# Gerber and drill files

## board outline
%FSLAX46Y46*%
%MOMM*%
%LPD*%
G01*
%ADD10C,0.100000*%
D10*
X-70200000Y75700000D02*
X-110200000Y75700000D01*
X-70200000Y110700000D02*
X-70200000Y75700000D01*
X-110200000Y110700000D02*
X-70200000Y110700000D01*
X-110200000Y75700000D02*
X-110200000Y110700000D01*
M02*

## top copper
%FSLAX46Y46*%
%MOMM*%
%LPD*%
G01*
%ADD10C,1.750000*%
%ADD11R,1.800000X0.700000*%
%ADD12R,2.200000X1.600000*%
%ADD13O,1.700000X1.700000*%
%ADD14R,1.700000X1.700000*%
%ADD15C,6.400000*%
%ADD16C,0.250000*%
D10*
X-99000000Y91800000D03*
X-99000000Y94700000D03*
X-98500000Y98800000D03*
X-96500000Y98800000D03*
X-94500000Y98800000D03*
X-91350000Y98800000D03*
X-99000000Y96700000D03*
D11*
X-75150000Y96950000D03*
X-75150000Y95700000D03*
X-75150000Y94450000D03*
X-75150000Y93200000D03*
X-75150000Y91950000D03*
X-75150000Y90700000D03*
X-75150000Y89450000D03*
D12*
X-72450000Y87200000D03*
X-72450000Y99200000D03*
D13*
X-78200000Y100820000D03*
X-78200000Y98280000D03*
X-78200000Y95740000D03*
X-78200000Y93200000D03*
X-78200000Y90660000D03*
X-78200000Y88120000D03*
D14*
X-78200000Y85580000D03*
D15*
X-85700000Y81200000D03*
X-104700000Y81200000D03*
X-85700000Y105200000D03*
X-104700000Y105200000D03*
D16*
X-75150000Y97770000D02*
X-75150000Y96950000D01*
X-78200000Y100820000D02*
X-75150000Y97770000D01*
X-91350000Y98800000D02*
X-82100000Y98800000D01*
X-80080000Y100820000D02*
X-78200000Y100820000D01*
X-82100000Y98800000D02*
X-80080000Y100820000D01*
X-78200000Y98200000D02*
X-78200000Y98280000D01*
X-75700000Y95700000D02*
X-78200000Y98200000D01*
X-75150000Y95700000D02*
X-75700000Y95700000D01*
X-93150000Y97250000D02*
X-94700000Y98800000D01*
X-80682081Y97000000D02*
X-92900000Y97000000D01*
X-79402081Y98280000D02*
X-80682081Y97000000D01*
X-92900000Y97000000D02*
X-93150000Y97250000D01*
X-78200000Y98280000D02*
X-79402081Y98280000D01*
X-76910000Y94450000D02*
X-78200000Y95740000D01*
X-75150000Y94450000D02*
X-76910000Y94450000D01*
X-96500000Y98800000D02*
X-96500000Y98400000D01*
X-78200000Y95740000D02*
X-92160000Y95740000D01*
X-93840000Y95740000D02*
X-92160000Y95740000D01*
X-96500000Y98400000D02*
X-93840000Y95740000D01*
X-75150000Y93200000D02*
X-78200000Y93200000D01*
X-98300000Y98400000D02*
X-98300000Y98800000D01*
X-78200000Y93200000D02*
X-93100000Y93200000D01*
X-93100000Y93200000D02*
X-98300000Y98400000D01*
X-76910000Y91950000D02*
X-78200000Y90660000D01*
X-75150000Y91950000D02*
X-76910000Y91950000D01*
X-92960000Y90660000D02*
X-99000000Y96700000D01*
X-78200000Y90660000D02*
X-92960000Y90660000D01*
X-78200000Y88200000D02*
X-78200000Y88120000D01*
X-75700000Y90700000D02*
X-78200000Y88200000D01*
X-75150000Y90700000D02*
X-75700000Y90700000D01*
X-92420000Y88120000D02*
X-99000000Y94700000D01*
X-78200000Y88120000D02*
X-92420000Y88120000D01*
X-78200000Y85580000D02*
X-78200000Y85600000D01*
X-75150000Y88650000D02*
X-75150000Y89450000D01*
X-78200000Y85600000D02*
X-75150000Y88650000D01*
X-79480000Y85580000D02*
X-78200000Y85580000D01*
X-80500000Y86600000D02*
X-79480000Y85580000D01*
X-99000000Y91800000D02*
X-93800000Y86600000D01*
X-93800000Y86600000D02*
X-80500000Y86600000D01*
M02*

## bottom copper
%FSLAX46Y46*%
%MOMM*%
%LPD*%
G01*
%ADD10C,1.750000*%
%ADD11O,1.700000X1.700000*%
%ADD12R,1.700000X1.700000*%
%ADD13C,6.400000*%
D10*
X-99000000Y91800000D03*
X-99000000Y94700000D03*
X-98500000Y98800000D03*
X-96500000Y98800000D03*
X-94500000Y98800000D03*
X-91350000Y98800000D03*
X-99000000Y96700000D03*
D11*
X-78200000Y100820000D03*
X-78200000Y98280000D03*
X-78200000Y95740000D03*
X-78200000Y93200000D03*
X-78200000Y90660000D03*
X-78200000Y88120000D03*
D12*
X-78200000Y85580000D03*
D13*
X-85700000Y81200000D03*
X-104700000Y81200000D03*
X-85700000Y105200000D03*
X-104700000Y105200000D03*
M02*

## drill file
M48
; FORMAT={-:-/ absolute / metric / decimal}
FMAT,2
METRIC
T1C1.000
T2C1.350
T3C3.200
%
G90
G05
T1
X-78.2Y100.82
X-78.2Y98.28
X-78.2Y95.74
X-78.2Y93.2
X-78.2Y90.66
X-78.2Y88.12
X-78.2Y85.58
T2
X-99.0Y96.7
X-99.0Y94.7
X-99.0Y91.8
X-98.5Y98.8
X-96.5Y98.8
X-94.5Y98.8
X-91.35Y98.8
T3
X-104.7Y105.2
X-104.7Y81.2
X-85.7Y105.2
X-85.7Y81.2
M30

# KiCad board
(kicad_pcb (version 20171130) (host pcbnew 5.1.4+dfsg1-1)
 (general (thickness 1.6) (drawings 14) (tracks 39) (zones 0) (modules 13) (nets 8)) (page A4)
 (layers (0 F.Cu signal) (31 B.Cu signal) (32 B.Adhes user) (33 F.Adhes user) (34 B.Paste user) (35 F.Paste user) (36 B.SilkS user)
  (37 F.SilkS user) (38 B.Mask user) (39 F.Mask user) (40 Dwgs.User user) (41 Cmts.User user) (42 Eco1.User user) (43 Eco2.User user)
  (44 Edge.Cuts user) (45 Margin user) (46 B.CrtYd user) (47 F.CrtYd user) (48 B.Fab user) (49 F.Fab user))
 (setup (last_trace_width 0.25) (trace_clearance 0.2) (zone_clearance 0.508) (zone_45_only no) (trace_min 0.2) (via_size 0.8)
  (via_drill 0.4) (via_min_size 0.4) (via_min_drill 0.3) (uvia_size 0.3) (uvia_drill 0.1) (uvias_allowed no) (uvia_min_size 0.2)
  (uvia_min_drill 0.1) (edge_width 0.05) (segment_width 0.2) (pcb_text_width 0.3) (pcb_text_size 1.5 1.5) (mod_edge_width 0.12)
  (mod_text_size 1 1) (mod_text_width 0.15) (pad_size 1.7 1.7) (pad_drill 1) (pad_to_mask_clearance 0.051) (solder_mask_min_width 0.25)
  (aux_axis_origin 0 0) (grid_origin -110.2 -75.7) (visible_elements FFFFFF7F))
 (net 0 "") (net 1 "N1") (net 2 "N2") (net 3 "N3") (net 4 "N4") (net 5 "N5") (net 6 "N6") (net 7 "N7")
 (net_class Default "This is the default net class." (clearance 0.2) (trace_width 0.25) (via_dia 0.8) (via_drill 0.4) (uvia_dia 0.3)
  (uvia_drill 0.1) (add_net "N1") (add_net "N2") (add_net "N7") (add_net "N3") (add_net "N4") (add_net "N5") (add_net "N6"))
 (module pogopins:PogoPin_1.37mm (layer F.Cu) (at -99 -91.8)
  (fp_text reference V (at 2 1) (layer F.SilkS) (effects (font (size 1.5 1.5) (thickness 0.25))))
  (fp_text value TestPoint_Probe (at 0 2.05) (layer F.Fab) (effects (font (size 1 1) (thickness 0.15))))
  (pad 1 thru_hole circle (at 0 0) (size 1.75 1.75) (drill 1.35) (layers *.Cu *.Mask) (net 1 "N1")))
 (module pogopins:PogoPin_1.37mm (layer F.Cu) (at -99 -94.7)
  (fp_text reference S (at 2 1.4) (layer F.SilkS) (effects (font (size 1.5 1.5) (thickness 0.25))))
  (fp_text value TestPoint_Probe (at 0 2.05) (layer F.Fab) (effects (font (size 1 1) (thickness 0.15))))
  (pad 1 thru_hole circle (at 0 0) (size 1.75 1.75) (drill 1.35) (layers *.Cu *.Mask) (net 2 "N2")))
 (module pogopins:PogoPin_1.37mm (layer F.Cu) (at -98.5 -98.8)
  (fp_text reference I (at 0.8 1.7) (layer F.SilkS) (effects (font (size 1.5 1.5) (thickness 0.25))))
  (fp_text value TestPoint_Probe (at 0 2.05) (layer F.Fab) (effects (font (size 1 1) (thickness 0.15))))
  (pad 1 thru_hole circle (at 0 0) (size 1.75 1.75) (drill 1.35) (layers *.Cu *.Mask) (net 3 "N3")))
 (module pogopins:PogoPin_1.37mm (layer F.Cu) (at -96.5 -98.8)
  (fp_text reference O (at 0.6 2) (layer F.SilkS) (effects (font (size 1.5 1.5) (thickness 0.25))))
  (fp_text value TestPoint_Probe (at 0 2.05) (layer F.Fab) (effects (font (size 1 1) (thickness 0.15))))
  (pad 1 thru_hole circle (at 0 0) (size 1.75 1.75) (drill 1.35) (layers *.Cu *.Mask) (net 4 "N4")))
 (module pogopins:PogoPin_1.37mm (layer F.Cu) (at -94.5 -98.8)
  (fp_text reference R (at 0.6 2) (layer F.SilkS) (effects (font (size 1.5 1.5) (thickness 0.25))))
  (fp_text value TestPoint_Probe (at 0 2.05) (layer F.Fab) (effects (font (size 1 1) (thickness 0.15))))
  (pad 1 thru_hole circle (at 0 0) (size 1.75 1.75) (drill 1.35) (layers *.Cu *.Mask) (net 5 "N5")))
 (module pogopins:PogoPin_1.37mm (layer F.Cu) (at -91.35 -98.8)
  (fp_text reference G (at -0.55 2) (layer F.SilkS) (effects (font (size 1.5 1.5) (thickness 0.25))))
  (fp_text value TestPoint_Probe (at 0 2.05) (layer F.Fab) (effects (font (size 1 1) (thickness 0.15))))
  (pad 1 thru_hole circle (at 0 0) (size 1.75 1.75) (drill 1.35) (layers *.Cu *.Mask) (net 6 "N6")))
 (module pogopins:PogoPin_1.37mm (layer F.Cu) (at -99 -96.7)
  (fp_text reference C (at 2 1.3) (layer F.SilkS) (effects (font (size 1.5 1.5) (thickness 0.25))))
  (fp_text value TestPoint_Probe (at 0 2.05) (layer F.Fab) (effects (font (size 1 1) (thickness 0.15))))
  (pad 1 thru_hole circle (at 0 0) (size 1.75 1.75) (drill 1.35) (layers *.Cu *.Mask) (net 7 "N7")))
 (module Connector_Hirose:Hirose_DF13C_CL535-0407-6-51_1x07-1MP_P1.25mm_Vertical (layer F.Cu) (at -73.7 -93.2 90)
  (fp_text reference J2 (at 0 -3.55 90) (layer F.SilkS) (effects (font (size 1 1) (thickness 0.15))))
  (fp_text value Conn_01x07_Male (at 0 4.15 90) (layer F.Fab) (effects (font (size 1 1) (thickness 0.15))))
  (pad 7 smd rect (at 3.75 -1.45 90) (size 0.7 1.8) (layers F.Cu F.Paste F.Mask) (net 6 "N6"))
  (pad 6 smd rect (at 2.5 -1.45 90) (size 0.7 1.8) (layers F.Cu F.Paste F.Mask) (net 5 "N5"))
  (pad 5 smd rect (at 1.25 -1.45 90) (size 0.7 1.8) (layers F.Cu F.Paste F.Mask) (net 4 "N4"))
  (pad 4 smd rect (at 0 -1.45 90) (size 0.7 1.8) (layers F.Cu F.Paste F.Mask) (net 3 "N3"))
  (pad 3 smd rect (at -1.25 -1.45 90) (size 0.7 1.8) (layers F.Cu F.Paste F.Mask) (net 7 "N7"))
  (pad 2 smd rect (at -2.5 -1.45 90) (size 0.7 1.8) (layers F.Cu F.Paste F.Mask) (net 2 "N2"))
  (pad 1 smd rect (at -3.75 -1.45 90) (size 0.7 1.8) (layers F.Cu F.Paste F.Mask) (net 1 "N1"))
  (pad MP smd rect (at -6 1.25 90) (size 1.6 2.2) (layers F.Cu F.Paste F.Mask))
  (pad MP smd rect (at 6 1.25 90) (size 1.6 2.2) (layers F.Cu F.Paste F.Mask)))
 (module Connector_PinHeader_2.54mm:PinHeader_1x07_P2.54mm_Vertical (layer F.Cu) (at -78.2 -85.58 180)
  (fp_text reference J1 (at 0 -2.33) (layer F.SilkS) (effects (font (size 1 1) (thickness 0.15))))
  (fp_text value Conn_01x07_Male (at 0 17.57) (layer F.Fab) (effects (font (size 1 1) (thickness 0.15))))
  (pad 7 thru_hole oval (at 0 15.24 180) (size 1.7 1.7) (drill 1) (layers *.Cu *.Mask) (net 6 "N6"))
  (pad 6 thru_hole oval (at 0 12.7 180) (size 1.7 1.7) (drill 1) (layers *.Cu *.Mask) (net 5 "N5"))
  (pad 5 thru_hole oval (at 0 10.16 180) (size 1.7 1.7) (drill 1) (layers *.Cu *.Mask) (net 4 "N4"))
  (pad 4 thru_hole oval (at 0 7.62 180) (size 1.7 1.7) (drill 1) (layers *.Cu *.Mask) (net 3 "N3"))
  (pad 3 thru_hole oval (at 0 5.08 180) (size 1.7 1.7) (drill 1) (layers *.Cu *.Mask) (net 7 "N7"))
  (pad 2 thru_hole oval (at 0 2.54 180) (size 1.7 1.7) (drill 1) (layers *.Cu *.Mask) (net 2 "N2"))
  (pad 1 thru_hole rect (at 0 0 180) (size 1.7 1.7) (drill 1) (layers *.Cu *.Mask) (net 1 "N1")))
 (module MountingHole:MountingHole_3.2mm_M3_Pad (layer F.Cu) (at -85.7 -81.2)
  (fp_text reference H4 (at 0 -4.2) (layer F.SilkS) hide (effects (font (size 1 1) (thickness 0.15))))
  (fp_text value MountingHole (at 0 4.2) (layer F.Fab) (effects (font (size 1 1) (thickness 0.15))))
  (pad 1 thru_hole circle (at 0 0) (size 6.4 6.4) (drill 3.2) (layers *.Cu *.Mask)))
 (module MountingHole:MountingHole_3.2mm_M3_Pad (layer F.Cu) (at -104.7 -81.2)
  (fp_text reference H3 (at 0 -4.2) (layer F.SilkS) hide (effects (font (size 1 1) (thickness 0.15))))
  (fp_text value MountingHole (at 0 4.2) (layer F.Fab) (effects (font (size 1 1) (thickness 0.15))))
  (pad 1 thru_hole circle (at 0 0) (size 6.4 6.4) (drill 3.2) (layers *.Cu *.Mask)))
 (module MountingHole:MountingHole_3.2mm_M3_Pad (layer F.Cu) (at -85.7 -105.2)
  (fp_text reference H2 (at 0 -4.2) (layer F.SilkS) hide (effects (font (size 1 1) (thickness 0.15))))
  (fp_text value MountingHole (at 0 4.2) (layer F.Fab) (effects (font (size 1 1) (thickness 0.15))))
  (pad 1 thru_hole circle (at 0 0) (size 6.4 6.4) (drill 3.2) (layers *.Cu *.Mask)))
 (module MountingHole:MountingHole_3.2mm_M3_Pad (layer F.Cu) (at -104.7 -105.2)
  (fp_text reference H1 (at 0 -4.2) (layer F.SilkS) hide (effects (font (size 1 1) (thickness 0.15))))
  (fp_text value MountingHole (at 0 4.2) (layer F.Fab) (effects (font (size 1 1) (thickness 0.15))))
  (pad 1 thru_hole circle (at 0 0) (size 6.4 6.4) (drill 3.2) (layers *.Cu *.Mask)))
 (gr_line (start -70.2 -75.7) (end -110.2 -75.7) (layer Edge.Cuts) (width 0.1))
 (gr_line (start -70.2 -110.7) (end -70.2 -75.7) (layer Edge.Cuts) (width 0.1))
 (gr_line (start -110.2 -110.7) (end -70.2 -110.7) (layer Edge.Cuts) (width 0.1))
 (gr_line (start -110.2 -75.7) (end -110.2 -110.7) (layer Edge.Cuts) (width 0.1))
 (segment (start -75.15 -97.77) (end -75.15 -96.95) (width 0.25) (layer F.Cu) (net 6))
 (segment (start -78.2 -100.82) (end -75.15 -97.77) (width 0.25) (layer F.Cu) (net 6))
 (segment (start -91.35 -98.8) (end -82.1 -98.8) (width 0.25) (layer F.Cu) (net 6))
 (segment (start -80.08 -100.82) (end -78.2 -100.82) (width 0.25) (layer F.Cu) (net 6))
 (segment (start -82.1 -98.8) (end -80.08 -100.82) (width 0.25) (layer F.Cu) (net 6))
 (segment (start -78.2 -98.2) (end -78.2 -98.28) (width 0.25) (layer F.Cu) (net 5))
 (segment (start -75.7 -95.7) (end -78.2 -98.2) (width 0.25) (layer F.Cu) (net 5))
 (segment (start -75.15 -95.7) (end -75.7 -95.7) (width 0.25) (layer F.Cu) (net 5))
 (segment (start -93.15 -97.25) (end -94.7 -98.8) (width 0.25) (layer F.Cu) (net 5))
 (segment (start -80.682081 -97) (end -92.9 -97) (width 0.25) (layer F.Cu) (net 5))
 (segment (start -79.402081 -98.28) (end -80.682081 -97) (width 0.25) (layer F.Cu) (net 5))
 (segment (start -92.9 -97) (end -93.15 -97.25) (width 0.25) (layer F.Cu) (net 5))
 (segment (start -78.2 -98.28) (end -79.402081 -98.28) (width 0.25) (layer F.Cu) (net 5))
 (segment (start -76.91 -94.45) (end -78.2 -95.74) (width 0.25) (layer F.Cu) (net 4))
 (segment (start -75.15 -94.45) (end -76.91 -94.45) (width 0.25) (layer F.Cu) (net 4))
 (segment (start -96.5 -98.8) (end -96.5 -98.4) (width 0.25) (layer F.Cu) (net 4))
 (segment (start -78.2 -95.74) (end -92.16 -95.74) (width 0.25) (layer F.Cu) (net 4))
 (segment (start -93.84 -95.74) (end -92.16 -95.74) (width 0.25) (layer F.Cu) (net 4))
 (segment (start -96.5 -98.4) (end -93.84 -95.74) (width 0.25) (layer F.Cu) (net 4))
 (segment (start -75.15 -93.2) (end -78.2 -93.2) (width 0.25) (layer F.Cu) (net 3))
 (segment (start -98.3 -98.4) (end -98.3 -98.8) (width 0.25) (layer F.Cu) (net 3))
 (segment (start -78.2 -93.2) (end -93.1 -93.2) (width 0.25) (layer F.Cu) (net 3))
 (segment (start -93.1 -93.2) (end -98.3 -98.4) (width 0.25) (layer F.Cu) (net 3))
 (segment (start -76.91 -91.95) (end -78.2 -90.66) (width 0.25) (layer F.Cu) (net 7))
 (segment (start -75.15 -91.95) (end -76.91 -91.95) (width 0.25) (layer F.Cu) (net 7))
 (segment (start -92.96 -90.66) (end -99 -96.7) (width 0.25) (layer F.Cu) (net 7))
 (segment (start -78.2 -90.66) (end -92.96 -90.66) (width 0.25) (layer F.Cu) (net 7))
 (segment (start -78.2 -88.2) (end -78.2 -88.12) (width 0.25) (layer F.Cu) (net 2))
 (segment (start -75.7 -90.7) (end -78.2 -88.2) (width 0.25) (layer F.Cu) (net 2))
 (segment (start -75.15 -90.7) (end -75.7 -90.7) (width 0.25) (layer F.Cu) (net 2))
 (segment (start -92.42 -88.12) (end -99 -94.7) (width 0.25) (layer F.Cu) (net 2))
 (segment (start -78.2 -88.12) (end -92.42 -88.12) (width 0.25) (layer F.Cu) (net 2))
 (segment (start -78.2 -85.58) (end -78.2 -85.6) (width 0.25) (layer F.Cu) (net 1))
 (segment (start -75.15 -88.65) (end -75.15 -89.45) (width 0.25) (layer F.Cu) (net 1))
 (segment (start -78.2 -85.6) (end -75.15 -88.65) (width 0.25) (layer F.Cu) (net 1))
 (segment (start -79.48 -85.58) (end -78.2 -85.58) (width 0.25) (layer F.Cu) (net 1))
 (segment (start -80.5 -86.6) (end -79.48 -85.58) (width 0.25) (layer F.Cu) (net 1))
 (segment (start -99 -91.8) (end -93.8 -86.6) (width 0.25) (layer F.Cu) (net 1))
 (segment (start -93.8 -86.6) (end -80.5 -86.6) (width 0.25) (layer F.Cu) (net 1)))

